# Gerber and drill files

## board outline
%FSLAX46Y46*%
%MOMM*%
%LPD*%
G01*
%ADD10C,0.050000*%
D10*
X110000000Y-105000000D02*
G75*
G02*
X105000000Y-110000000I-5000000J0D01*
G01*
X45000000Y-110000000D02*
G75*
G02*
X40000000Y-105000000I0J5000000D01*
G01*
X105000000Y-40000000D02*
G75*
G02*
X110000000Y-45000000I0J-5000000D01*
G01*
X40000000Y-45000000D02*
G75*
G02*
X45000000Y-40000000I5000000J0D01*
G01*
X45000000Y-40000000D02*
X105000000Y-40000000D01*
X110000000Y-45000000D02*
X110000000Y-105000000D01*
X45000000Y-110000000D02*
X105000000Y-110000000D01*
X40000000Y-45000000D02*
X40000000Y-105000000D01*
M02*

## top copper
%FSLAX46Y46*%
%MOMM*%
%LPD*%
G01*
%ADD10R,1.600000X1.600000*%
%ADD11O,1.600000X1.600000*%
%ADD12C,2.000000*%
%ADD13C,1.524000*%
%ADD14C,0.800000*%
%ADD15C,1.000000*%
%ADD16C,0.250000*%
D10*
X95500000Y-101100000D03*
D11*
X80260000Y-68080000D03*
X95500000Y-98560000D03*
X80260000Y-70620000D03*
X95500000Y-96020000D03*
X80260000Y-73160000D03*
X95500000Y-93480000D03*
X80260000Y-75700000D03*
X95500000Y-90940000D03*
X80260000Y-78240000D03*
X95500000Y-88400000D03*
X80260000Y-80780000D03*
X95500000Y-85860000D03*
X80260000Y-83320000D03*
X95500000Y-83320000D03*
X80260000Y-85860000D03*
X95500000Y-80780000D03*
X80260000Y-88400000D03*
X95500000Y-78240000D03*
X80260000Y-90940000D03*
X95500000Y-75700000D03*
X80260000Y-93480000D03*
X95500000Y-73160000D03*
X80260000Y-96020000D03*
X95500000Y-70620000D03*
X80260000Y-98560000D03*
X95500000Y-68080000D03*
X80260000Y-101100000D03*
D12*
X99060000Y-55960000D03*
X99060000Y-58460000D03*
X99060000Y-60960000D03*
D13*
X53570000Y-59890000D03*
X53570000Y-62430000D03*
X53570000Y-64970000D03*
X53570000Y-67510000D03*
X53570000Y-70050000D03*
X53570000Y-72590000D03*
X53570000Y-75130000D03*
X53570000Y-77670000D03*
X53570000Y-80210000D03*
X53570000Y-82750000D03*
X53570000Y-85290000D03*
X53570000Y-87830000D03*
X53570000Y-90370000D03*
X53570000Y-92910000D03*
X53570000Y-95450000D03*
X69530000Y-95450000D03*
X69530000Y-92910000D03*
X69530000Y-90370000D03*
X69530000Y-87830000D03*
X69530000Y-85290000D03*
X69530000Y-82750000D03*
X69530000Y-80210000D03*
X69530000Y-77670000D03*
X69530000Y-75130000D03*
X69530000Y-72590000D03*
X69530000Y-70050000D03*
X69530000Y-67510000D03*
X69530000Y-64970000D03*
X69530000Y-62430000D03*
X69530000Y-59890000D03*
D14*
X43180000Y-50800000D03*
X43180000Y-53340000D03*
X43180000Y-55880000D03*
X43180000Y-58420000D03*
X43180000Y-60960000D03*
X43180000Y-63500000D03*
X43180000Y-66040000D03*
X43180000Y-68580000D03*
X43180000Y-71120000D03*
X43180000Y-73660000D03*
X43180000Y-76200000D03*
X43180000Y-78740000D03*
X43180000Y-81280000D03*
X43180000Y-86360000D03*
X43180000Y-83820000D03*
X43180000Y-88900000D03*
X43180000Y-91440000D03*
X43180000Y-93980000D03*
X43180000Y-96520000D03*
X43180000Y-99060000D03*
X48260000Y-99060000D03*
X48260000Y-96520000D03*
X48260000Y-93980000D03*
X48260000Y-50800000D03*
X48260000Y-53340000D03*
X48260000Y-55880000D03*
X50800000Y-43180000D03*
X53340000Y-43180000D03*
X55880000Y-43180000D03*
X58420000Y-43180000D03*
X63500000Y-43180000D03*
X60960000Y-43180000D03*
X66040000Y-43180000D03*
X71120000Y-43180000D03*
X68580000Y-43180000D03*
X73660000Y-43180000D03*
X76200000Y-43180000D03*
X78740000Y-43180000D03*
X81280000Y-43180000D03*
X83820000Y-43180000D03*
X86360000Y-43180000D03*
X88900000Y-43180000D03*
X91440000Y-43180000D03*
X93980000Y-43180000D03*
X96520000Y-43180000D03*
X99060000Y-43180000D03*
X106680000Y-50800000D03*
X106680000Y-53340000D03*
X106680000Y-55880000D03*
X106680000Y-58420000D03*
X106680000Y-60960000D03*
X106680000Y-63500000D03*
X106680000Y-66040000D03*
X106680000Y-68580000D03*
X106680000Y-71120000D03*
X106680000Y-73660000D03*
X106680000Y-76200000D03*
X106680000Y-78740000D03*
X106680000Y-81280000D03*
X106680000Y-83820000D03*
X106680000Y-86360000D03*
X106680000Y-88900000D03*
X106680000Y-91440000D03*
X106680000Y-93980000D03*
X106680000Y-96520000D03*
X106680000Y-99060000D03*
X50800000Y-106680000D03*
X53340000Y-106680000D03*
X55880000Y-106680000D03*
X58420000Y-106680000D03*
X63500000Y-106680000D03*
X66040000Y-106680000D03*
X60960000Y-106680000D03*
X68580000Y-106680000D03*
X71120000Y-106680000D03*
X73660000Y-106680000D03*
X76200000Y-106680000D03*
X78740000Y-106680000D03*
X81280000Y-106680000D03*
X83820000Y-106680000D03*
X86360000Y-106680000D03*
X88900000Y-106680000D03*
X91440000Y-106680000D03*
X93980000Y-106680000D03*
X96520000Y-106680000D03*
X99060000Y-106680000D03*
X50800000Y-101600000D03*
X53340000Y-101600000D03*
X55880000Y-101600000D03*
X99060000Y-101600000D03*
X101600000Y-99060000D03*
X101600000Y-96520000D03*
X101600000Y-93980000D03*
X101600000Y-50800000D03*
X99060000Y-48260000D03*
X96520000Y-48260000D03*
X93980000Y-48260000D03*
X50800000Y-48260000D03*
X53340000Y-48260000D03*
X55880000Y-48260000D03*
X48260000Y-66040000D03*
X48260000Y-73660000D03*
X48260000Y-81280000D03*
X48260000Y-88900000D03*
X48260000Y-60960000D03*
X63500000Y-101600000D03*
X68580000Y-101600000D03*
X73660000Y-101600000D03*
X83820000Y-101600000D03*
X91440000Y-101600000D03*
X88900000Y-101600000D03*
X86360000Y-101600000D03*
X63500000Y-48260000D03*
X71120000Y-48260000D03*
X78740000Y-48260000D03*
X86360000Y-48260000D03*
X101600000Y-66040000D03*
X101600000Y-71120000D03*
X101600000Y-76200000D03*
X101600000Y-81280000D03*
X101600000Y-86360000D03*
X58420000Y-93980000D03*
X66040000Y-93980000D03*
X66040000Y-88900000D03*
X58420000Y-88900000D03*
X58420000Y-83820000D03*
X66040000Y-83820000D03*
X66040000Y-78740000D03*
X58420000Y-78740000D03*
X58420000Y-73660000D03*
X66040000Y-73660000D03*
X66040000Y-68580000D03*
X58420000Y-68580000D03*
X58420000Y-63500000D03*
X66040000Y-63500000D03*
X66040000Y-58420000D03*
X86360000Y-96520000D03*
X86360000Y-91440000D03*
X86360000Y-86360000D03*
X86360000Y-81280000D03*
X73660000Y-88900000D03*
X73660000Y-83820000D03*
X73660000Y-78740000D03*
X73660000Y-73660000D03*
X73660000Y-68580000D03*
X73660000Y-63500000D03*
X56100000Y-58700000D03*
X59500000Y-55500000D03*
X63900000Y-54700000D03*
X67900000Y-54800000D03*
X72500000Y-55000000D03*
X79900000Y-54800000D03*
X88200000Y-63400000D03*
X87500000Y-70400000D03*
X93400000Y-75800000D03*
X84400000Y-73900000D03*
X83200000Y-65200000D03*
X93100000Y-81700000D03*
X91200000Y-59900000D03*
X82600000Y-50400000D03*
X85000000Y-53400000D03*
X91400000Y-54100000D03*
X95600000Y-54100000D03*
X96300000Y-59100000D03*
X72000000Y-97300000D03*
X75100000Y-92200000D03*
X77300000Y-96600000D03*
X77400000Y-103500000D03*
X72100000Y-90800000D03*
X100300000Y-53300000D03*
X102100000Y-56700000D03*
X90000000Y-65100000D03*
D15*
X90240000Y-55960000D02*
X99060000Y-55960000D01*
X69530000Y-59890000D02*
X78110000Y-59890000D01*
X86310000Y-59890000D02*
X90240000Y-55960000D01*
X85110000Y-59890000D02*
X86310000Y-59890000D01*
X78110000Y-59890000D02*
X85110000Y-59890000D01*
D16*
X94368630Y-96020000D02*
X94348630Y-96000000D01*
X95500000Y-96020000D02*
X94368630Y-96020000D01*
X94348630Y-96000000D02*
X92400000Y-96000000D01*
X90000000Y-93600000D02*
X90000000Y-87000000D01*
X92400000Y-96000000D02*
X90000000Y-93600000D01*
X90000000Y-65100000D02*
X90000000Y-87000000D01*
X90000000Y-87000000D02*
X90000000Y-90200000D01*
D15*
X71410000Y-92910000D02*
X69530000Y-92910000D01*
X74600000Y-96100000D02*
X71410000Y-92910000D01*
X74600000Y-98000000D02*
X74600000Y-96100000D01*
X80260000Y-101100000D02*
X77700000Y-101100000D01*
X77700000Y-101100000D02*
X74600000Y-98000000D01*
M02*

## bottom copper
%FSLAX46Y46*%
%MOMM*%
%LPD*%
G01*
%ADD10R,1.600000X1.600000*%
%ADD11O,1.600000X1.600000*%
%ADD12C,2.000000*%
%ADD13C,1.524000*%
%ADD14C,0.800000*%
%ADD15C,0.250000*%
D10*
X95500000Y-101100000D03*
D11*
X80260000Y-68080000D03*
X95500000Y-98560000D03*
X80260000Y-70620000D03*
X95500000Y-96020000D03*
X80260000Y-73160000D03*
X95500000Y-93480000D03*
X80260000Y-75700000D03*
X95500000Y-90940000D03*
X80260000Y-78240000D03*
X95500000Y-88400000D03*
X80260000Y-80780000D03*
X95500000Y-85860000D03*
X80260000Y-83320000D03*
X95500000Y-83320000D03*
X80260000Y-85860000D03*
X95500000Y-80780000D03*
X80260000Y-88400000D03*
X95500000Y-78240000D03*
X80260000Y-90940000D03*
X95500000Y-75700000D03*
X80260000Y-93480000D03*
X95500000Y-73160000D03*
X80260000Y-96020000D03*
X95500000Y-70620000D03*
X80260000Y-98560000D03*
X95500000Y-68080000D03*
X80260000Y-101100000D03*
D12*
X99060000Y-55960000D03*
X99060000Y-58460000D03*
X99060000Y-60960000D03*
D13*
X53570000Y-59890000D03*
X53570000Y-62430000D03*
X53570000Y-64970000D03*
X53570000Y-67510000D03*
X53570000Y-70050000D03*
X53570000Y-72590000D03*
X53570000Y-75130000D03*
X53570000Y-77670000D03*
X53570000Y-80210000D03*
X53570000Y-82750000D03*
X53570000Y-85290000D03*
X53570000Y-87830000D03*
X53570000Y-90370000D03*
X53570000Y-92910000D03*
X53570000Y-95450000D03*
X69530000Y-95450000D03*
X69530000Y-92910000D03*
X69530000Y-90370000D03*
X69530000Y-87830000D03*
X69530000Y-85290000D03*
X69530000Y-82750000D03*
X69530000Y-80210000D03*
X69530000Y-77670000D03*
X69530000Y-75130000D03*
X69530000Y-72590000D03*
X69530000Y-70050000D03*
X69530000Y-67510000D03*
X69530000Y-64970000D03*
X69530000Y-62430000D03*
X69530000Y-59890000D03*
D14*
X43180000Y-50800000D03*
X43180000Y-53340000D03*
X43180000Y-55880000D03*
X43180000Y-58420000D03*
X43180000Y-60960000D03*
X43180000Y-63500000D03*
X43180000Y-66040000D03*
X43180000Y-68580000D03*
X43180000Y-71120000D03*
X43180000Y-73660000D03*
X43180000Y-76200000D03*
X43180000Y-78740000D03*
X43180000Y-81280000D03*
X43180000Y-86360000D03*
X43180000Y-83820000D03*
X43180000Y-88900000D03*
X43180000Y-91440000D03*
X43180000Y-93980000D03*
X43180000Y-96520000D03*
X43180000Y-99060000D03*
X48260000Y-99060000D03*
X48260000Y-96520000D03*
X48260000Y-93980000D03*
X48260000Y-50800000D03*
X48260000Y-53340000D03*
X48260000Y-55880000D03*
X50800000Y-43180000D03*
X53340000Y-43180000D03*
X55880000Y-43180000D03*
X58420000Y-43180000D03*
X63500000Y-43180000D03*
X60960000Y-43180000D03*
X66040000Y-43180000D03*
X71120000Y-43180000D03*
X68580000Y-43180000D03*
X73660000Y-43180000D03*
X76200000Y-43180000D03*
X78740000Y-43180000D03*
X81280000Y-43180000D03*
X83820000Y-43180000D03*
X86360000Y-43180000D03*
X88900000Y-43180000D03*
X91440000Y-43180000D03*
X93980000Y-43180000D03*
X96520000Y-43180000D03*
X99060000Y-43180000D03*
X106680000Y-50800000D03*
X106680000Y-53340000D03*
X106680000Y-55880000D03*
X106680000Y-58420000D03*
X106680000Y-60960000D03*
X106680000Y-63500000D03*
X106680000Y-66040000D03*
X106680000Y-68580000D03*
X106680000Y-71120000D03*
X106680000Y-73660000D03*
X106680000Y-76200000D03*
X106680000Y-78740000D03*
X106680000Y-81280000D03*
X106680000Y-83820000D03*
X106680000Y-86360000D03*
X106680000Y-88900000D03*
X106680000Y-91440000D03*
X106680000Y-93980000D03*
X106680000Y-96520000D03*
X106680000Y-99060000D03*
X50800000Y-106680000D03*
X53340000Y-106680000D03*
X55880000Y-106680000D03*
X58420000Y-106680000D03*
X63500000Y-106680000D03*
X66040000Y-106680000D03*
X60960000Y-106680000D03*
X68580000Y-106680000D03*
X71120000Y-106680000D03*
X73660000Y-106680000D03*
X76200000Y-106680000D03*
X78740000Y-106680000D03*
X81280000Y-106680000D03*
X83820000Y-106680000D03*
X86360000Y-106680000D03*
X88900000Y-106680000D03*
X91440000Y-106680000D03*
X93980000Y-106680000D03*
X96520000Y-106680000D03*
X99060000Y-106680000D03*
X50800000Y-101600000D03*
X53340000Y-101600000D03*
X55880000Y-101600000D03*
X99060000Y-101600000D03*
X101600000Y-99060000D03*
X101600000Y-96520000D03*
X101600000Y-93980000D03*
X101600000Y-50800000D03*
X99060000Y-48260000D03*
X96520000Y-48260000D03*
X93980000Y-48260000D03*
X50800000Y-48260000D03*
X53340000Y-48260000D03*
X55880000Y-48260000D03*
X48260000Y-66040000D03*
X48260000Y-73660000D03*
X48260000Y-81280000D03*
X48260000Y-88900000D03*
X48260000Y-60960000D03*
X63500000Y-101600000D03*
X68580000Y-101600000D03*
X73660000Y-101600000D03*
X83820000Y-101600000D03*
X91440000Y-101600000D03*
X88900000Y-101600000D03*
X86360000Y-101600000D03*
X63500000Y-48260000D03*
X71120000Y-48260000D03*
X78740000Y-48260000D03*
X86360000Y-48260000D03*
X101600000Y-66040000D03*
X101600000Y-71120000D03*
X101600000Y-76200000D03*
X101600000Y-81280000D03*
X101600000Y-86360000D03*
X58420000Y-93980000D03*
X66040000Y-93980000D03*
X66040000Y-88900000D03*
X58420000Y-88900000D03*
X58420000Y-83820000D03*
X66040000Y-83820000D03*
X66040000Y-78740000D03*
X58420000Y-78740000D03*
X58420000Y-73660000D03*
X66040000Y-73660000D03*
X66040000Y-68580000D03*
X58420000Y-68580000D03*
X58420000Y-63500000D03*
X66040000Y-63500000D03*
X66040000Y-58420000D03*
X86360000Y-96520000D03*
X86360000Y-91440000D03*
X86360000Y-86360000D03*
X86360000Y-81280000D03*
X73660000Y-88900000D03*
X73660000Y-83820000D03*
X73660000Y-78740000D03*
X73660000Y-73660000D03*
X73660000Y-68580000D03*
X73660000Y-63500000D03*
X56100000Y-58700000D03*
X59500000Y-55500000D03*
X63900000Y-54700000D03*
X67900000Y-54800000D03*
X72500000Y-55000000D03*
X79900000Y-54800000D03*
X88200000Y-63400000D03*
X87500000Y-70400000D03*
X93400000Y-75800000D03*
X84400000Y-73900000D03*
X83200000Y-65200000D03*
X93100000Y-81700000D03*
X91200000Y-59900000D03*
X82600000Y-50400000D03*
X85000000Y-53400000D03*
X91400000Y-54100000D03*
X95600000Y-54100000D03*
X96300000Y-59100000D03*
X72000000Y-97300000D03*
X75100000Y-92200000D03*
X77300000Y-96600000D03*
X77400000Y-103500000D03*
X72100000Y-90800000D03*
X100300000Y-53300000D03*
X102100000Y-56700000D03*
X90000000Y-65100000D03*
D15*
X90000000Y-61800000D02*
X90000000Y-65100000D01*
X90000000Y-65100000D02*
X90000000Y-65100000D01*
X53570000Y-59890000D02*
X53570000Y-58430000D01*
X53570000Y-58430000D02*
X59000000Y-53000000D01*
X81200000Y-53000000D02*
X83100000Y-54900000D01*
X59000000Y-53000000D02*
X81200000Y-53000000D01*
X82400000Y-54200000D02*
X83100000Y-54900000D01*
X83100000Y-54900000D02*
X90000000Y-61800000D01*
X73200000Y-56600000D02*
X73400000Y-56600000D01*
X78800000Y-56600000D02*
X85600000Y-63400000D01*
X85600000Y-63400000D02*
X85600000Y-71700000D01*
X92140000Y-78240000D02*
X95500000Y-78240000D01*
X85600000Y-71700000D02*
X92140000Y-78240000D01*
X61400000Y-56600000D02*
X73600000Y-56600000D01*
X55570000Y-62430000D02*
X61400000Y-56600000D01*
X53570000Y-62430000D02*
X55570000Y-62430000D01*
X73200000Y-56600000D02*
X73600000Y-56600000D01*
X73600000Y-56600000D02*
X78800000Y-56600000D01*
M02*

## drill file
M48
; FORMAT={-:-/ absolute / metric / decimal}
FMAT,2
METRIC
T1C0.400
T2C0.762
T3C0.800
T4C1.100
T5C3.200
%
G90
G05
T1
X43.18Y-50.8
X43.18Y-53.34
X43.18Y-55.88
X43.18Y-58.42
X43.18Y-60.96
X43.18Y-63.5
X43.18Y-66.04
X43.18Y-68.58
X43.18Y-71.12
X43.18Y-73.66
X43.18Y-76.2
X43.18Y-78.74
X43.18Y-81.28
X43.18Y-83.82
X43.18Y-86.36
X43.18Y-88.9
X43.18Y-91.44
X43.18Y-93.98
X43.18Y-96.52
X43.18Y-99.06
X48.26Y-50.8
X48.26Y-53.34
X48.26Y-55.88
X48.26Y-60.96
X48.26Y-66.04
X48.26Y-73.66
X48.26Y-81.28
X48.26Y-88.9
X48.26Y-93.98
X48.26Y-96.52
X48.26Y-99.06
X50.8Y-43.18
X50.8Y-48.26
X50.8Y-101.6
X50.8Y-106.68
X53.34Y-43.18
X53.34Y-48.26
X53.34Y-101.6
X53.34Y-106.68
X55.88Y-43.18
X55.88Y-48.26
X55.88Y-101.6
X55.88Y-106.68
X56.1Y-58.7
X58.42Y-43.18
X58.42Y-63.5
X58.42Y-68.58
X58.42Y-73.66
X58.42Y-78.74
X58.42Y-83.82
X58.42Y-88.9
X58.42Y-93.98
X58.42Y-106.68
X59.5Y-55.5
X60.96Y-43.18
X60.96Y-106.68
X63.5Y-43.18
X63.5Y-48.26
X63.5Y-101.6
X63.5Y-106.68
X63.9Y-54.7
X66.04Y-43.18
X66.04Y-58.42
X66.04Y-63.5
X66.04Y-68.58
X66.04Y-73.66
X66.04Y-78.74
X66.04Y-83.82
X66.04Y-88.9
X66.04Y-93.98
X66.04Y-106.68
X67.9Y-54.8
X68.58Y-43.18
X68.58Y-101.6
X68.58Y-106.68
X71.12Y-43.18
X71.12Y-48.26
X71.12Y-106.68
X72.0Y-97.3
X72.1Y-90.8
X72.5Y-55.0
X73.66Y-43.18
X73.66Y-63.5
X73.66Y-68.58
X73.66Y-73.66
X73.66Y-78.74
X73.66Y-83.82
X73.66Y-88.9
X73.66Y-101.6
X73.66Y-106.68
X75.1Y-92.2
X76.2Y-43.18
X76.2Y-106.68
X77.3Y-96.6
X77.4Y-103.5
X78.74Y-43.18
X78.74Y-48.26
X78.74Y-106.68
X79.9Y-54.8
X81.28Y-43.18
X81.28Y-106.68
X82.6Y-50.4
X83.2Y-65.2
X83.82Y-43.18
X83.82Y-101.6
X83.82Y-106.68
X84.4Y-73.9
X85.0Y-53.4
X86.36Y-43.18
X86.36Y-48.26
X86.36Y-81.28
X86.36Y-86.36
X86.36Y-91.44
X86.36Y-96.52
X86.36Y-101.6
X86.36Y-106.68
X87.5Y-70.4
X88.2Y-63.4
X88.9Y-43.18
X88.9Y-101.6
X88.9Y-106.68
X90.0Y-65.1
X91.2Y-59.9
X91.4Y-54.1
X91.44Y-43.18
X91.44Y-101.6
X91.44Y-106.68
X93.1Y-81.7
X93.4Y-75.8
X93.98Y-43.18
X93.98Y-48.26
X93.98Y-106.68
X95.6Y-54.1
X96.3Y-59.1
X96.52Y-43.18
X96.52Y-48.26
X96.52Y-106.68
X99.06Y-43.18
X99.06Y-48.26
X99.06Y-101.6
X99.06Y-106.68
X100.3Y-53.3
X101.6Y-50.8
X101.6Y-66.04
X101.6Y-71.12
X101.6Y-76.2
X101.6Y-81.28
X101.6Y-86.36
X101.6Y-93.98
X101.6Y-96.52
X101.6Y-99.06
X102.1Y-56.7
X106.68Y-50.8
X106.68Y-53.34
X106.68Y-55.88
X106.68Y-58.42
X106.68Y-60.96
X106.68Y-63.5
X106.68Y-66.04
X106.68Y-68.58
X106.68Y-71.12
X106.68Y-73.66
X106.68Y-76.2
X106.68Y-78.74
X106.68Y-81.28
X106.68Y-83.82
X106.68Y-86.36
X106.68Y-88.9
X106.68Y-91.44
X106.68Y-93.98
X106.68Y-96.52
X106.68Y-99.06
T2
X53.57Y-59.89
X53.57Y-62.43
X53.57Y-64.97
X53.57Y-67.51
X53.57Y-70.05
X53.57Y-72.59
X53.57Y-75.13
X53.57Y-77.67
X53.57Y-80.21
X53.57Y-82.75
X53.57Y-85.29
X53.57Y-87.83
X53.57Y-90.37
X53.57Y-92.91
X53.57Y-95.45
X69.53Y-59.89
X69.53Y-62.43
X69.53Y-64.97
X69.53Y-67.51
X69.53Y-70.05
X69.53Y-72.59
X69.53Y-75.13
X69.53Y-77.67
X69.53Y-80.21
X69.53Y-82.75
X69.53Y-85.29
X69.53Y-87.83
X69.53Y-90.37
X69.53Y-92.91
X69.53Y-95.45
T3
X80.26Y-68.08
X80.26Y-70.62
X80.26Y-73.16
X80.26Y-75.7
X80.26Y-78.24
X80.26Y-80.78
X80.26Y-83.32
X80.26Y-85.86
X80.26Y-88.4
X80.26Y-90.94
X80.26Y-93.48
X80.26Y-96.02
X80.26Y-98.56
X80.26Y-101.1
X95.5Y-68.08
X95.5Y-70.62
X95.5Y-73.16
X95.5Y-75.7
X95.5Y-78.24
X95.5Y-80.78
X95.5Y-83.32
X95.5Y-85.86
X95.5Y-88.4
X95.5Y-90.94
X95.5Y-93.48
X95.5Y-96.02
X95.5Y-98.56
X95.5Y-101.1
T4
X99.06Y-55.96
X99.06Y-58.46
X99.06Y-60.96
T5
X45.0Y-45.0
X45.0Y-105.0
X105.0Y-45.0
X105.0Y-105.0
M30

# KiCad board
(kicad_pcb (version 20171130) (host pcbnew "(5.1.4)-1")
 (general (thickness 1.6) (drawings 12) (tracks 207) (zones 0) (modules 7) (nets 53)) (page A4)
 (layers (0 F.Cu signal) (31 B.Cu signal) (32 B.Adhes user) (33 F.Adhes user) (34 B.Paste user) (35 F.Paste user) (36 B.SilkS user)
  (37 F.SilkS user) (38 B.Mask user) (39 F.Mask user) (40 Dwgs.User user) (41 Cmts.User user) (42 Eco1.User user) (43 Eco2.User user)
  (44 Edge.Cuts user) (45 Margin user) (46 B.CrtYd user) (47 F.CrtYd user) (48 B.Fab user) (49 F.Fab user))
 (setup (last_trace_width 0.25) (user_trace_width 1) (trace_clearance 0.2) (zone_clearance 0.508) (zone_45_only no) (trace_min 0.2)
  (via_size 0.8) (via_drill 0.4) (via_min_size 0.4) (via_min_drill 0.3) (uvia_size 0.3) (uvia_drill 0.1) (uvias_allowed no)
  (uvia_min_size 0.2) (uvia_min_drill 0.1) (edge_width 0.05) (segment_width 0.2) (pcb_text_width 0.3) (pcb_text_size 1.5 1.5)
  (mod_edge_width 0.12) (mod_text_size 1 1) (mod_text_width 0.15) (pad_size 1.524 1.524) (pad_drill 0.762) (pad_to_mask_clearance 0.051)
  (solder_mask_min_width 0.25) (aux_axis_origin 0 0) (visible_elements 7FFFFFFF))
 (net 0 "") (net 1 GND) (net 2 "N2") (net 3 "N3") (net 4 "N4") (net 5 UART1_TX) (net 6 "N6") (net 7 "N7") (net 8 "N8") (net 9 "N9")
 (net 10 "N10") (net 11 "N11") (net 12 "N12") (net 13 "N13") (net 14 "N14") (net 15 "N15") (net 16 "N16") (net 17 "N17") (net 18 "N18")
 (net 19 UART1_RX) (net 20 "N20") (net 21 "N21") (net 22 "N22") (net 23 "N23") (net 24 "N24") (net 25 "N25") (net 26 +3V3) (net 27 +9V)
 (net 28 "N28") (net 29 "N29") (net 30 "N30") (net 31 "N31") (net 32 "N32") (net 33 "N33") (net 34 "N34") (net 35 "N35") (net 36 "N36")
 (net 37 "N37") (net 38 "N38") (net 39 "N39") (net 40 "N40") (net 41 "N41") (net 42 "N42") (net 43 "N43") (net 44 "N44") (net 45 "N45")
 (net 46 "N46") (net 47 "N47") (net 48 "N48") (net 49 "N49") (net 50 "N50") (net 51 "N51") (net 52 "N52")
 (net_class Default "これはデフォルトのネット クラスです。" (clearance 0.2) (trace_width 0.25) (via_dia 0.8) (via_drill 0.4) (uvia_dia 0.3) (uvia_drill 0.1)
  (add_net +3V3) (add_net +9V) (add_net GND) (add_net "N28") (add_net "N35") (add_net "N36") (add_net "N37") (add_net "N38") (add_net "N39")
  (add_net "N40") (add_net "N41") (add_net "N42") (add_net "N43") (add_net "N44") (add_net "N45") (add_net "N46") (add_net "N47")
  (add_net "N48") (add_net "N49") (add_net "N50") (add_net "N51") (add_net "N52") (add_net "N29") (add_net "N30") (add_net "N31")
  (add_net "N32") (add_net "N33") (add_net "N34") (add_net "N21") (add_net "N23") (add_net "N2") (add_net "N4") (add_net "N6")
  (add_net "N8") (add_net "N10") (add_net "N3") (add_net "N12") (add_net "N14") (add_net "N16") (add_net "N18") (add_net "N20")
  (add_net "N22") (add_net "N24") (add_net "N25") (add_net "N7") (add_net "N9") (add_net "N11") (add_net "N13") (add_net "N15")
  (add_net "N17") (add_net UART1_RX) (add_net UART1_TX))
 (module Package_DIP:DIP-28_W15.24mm (layer F.Cu) (at 95.5 101.1 180)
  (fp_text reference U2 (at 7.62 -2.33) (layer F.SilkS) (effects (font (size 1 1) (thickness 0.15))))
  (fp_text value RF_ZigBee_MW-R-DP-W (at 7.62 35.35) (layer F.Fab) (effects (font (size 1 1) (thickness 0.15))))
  (pad 1 thru_hole rect (at 0 0 180) (size 1.6 1.6) (drill 0.8) (layers *.Cu *.Mask) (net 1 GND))
  (pad 15 thru_hole oval (at 15.24 33.02 180) (size 1.6 1.6) (drill 0.8) (layers *.Cu *.Mask) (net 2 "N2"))
  (pad 2 thru_hole oval (at 0 2.54 180) (size 1.6 1.6) (drill 0.8) (layers *.Cu *.Mask) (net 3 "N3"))
  (pad 16 thru_hole oval (at 15.24 30.48 180) (size 1.6 1.6) (drill 0.8) (layers *.Cu *.Mask) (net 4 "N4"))
  (pad 3 thru_hole oval (at 0 5.08 180) (size 1.6 1.6) (drill 0.8) (layers *.Cu *.Mask) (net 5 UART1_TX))
  (pad 17 thru_hole oval (at 15.24 27.94 180) (size 1.6 1.6) (drill 0.8) (layers *.Cu *.Mask) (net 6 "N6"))
  (pad 4 thru_hole oval (at 0 7.62 180) (size 1.6 1.6) (drill 0.8) (layers *.Cu *.Mask) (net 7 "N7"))
  (pad 18 thru_hole oval (at 15.24 25.4 180) (size 1.6 1.6) (drill 0.8) (layers *.Cu *.Mask) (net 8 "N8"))
  (pad 5 thru_hole oval (at 0 10.16 180) (size 1.6 1.6) (drill 0.8) (layers *.Cu *.Mask) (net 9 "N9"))
  (pad 19 thru_hole oval (at 15.24 22.86 180) (size 1.6 1.6) (drill 0.8) (layers *.Cu *.Mask) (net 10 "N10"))
  (pad 6 thru_hole oval (at 0 12.7 180) (size 1.6 1.6) (drill 0.8) (layers *.Cu *.Mask) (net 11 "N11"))
  (pad 20 thru_hole oval (at 15.24 20.32 180) (size 1.6 1.6) (drill 0.8) (layers *.Cu *.Mask) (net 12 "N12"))
  (pad 7 thru_hole oval (at 0 15.24 180) (size 1.6 1.6) (drill 0.8) (layers *.Cu *.Mask) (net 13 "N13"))
  (pad 21 thru_hole oval (at 15.24 17.78 180) (size 1.6 1.6) (drill 0.8) (layers *.Cu *.Mask) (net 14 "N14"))
  (pad 8 thru_hole oval (at 0 17.78 180) (size 1.6 1.6) (drill 0.8) (layers *.Cu *.Mask) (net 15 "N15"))
  (pad 22 thru_hole oval (at 15.24 15.24 180) (size 1.6 1.6) (drill 0.8) (layers *.Cu *.Mask) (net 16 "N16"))
  (pad 9 thru_hole oval (at 0 20.32 180) (size 1.6 1.6) (drill 0.8) (layers *.Cu *.Mask) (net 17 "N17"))
  (pad 23 thru_hole oval (at 15.24 12.7 180) (size 1.6 1.6) (drill 0.8) (layers *.Cu *.Mask) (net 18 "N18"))
  (pad 10 thru_hole oval (at 0 22.86 180) (size 1.6 1.6) (drill 0.8) (layers *.Cu *.Mask) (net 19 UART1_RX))
  (pad 24 thru_hole oval (at 15.24 10.16 180) (size 1.6 1.6) (drill 0.8) (layers *.Cu *.Mask) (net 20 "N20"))
  (pad 11 thru_hole oval (at 0 25.4 180) (size 1.6 1.6) (drill 0.8) (layers *.Cu *.Mask) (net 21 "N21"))
  (pad 25 thru_hole oval (at 15.24 7.62 180) (size 1.6 1.6) (drill 0.8) (layers *.Cu *.Mask) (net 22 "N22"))
  (pad 12 thru_hole oval (at 0 27.94 180) (size 1.6 1.6) (drill 0.8) (layers *.Cu *.Mask) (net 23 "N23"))
  (pad 26 thru_hole oval (at 15.24 5.08 180) (size 1.6 1.6) (drill 0.8) (layers *.Cu *.Mask) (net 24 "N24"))
  (pad 13 thru_hole oval (at 0 30.48 180) (size 1.6 1.6) (drill 0.8) (layers *.Cu *.Mask) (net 1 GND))
  (pad 27 thru_hole oval (at 15.24 2.54 180) (size 1.6 1.6) (drill 0.8) (layers *.Cu *.Mask) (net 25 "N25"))
  (pad 14 thru_hole oval (at 0 33.02 180) (size 1.6 1.6) (drill 0.8) (layers *.Cu *.Mask) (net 1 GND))
  (pad 28 thru_hole oval (at 15.24 0 180) (size 1.6 1.6) (drill 0.8) (layers *.Cu *.Mask) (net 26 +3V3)))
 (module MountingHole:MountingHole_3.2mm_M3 (layer F.Cu) (at 45 45)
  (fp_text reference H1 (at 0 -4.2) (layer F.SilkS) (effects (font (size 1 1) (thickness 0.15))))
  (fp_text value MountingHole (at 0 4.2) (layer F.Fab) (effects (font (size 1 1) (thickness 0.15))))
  (pad 1 np_thru_hole circle (at 0 0) (size 3.2 3.2) (drill 3.2) (layers *.Cu *.Mask)))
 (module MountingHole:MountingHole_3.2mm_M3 (layer F.Cu) (at 105 45)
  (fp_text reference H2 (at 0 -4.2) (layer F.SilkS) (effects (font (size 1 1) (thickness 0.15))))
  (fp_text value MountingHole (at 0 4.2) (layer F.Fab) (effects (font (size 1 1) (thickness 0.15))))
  (pad 1 np_thru_hole circle (at 0 0) (size 3.2 3.2) (drill 3.2) (layers *.Cu *.Mask)))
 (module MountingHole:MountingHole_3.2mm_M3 (layer F.Cu) (at 45 105)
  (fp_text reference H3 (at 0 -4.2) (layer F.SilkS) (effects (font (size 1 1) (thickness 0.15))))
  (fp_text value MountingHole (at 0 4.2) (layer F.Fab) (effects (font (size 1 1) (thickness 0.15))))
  (pad 1 np_thru_hole circle (at 0 0) (size 3.2 3.2) (drill 3.2) (layers *.Cu *.Mask)))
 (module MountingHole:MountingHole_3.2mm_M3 (layer F.Cu) (at 105 105)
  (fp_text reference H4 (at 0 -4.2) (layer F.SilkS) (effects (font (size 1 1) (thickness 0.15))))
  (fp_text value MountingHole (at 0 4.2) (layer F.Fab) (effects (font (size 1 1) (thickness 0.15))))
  (pad 1 np_thru_hole circle (at 0 0) (size 3.2 3.2) (drill 3.2) (layers *.Cu *.Mask)))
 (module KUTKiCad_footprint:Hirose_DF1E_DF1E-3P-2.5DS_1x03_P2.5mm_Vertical (layer F.Cu) (at 99.06 55.96 270)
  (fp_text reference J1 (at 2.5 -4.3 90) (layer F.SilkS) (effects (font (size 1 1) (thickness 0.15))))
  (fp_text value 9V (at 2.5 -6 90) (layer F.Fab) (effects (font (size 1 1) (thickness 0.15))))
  (pad 1 thru_hole circle (at 0 0 270) (size 2 2) (drill 1.1) (layers *.Cu *.Mask) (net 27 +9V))
  (pad 2 thru_hole circle (at 2.5 0 270) (size 2 2) (drill 1.1) (layers *.Cu *.Mask) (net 1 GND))
  (pad 3 thru_hole circle (at 5 0 270) (size 2 2) (drill 1.1) (layers *.Cu *.Mask) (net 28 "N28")))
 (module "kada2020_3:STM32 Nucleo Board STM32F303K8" (layer F.Cu) (at 52.3 51)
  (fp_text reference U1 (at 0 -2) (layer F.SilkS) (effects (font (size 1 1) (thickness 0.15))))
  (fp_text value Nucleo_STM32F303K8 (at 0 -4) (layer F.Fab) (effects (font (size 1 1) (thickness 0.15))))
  (pad 1 thru_hole circle (at 1.27 8.89) (size 1.524 1.524) (drill 0.762) (layers *.Cu *.Mask) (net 5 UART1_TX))
  (pad 2 thru_hole circle (at 1.27 11.43) (size 1.524 1.524) (drill 0.762) (layers *.Cu *.Mask) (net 19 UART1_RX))
  (pad 3 thru_hole circle (at 1.27 13.97) (size 1.524 1.524) (drill 0.762) (layers *.Cu *.Mask) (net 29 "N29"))
  (pad 4 thru_hole circle (at 1.27 16.51) (size 1.524 1.524) (drill 0.762) (layers *.Cu *.Mask) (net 1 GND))
  (pad 5 thru_hole circle (at 1.27 19.05) (size 1.524 1.524) (drill 0.762) (layers *.Cu *.Mask) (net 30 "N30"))
  (pad 6 thru_hole circle (at 1.27 21.59) (size 1.524 1.524) (drill 0.762) (layers *.Cu *.Mask) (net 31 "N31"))
  (pad 7 thru_hole circle (at 1.27 24.13) (size 1.524 1.524) (drill 0.762) (layers *.Cu *.Mask) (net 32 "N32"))
  (pad 8 thru_hole circle (at 1.27 26.67) (size 1.524 1.524) (drill 0.762) (layers *.Cu *.Mask) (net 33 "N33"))
  (pad 9 thru_hole circle (at 1.27 29.21) (size 1.524 1.524) (drill 0.762) (layers *.Cu *.Mask) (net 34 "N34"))
  (pad 10 thru_hole circle (at 1.27 31.75) (size 1.524 1.524) (drill 0.762) (layers *.Cu *.Mask) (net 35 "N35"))
  (pad 11 thru_hole circle (at 1.27 34.29) (size 1.524 1.524) (drill 0.762) (layers *.Cu *.Mask) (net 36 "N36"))
  (pad 12 thru_hole circle (at 1.27 36.83) (size 1.524 1.524) (drill 0.762) (layers *.Cu *.Mask) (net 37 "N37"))
  (pad 13 thru_hole circle (at 1.27 39.37) (size 1.524 1.524) (drill 0.762) (layers *.Cu *.Mask) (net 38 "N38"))
  (pad 14 thru_hole circle (at 1.27 41.91) (size 1.524 1.524) (drill 0.762) (layers *.Cu *.Mask) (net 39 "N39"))
  (pad 15 thru_hole circle (at 1.27 44.45) (size 1.524 1.524) (drill 0.762) (layers *.Cu *.Mask) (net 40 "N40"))
  (pad 16 thru_hole circle (at 17.23 44.45) (size 1.524 1.524) (drill 0.762) (layers *.Cu *.Mask) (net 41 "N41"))
  (pad 17 thru_hole circle (at 17.23 41.91) (size 1.524 1.524) (drill 0.762) (layers *.Cu *.Mask) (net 26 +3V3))
  (pad 18 thru_hole circle (at 17.23 39.37) (size 1.524 1.524) (drill 0.762) (layers *.Cu *.Mask) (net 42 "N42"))
  (pad 19 thru_hole circle (at 17.23 36.83) (size 1.524 1.524) (drill 0.762) (layers *.Cu *.Mask) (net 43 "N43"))
  (pad 20 thru_hole circle (at 17.23 34.29) (size 1.524 1.524) (drill 0.762) (layers *.Cu *.Mask) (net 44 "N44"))
  (pad 21 thru_hole circle (at 17.23 31.75) (size 1.524 1.524) (drill 0.762) (layers *.Cu *.Mask) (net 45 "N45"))
  (pad 22 thru_hole circle (at 17.23 29.21) (size 1.524 1.524) (drill 0.762) (layers *.Cu *.Mask) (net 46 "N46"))
  (pad 23 thru_hole circle (at 17.23 26.67) (size 1.524 1.524) (drill 0.762) (layers *.Cu *.Mask) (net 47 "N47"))
  (pad 24 thru_hole circle (at 17.23 24.13) (size 1.524 1.524) (drill 0.762) (layers *.Cu *.Mask) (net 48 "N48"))
  (pad 25 thru_hole circle (at 17.23 21.59) (size 1.524 1.524) (drill 0.762) (layers *.Cu *.Mask) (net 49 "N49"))
  (pad 26 thru_hole circle (at 17.23 19.05) (size 1.524 1.524) (drill 0.762) (layers *.Cu *.Mask) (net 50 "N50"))
  (pad 27 thru_hole circle (at 17.23 16.51) (size 1.524 1.524) (drill 0.762) (layers *.Cu *.Mask) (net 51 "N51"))
  (pad 28 thru_hole circle (at 17.23 13.97) (size 1.524 1.524) (drill 0.762) (layers *.Cu *.Mask) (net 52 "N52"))
  (pad 29 thru_hole circle (at 17.23 11.43) (size 1.524 1.524) (drill 0.762) (layers *.Cu *.Mask) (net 1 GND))
  (pad 30 thru_hole circle (at 17.23 8.89) (size 1.524 1.524) (drill 0.762) (layers *.Cu *.Mask) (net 27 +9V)))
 (gr_arc (start 105 105) (end 105 110) (angle -90) (layer Edge.Cuts) (width 0.05))
 (gr_arc (start 45 105) (end 40 105) (angle -90) (layer Edge.Cuts) (width 0.05))
 (gr_arc (start 105 45) (end 110 45) (angle -90) (layer Edge.Cuts) (width 0.05))
 (gr_arc (start 45 45) (end 45 40) (angle -90) (layer Edge.Cuts) (width 0.05))
 (gr_line (start 45 40) (end 105 40) (layer Edge.Cuts) (width 0.05))
 (gr_line (start 110 45) (end 110 105) (layer Edge.Cuts) (width 0.05))
 (gr_line (start 45 110) (end 105 110) (layer Edge.Cuts) (width 0.05))
 (gr_line (start 40 45) (end 40 105) (layer Edge.Cuts) (width 0.05))
 (segment (start 90.24 55.96) (end 99.06 55.96) (width 1) (layer F.Cu) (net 27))
 (segment (start 69.53 59.89) (end 78.11 59.89) (width 1) (layer F.Cu) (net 27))
 (segment (start 86.31 59.89) (end 90.24 55.96) (width 1) (layer F.Cu) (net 27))
 (segment (start 85.11 59.89) (end 86.31 59.89) (width 1) (layer F.Cu) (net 27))
 (segment (start 78.11 59.89) (end 85.11 59.89) (width 1) (layer F.Cu) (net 27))
 (via (at 43.18 50.8) (size 0.8) (drill 0.4) (layers F.Cu B.Cu) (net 1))
 (via (at 43.18 53.34) (size 0.8) (drill 0.4) (layers F.Cu B.Cu) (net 1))
 (via (at 43.18 55.88) (size 0.8) (drill 0.4) (layers F.Cu B.Cu) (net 1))
 (via (at 43.18 58.42) (size 0.8) (drill 0.4) (layers F.Cu B.Cu) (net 1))
 (via (at 43.18 60.96) (size 0.8) (drill 0.4) (layers F.Cu B.Cu) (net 1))
 (via (at 43.18 63.5) (size 0.8) (drill 0.4) (layers F.Cu B.Cu) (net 1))
 (via (at 43.18 66.04) (size 0.8) (drill 0.4) (layers F.Cu B.Cu) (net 1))
 (via (at 43.18 68.58) (size 0.8) (drill 0.4) (layers F.Cu B.Cu) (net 1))
 (via (at 43.18 71.12) (size 0.8) (drill 0.4) (layers F.Cu B.Cu) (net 1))
 (via (at 43.18 73.66) (size 0.8) (drill 0.4) (layers F.Cu B.Cu) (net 1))
 (via (at 43.18 76.2) (size 0.8) (drill 0.4) (layers F.Cu B.Cu) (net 1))
 (via (at 43.18 78.74) (size 0.8) (drill 0.4) (layers F.Cu B.Cu) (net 1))
 (via (at 43.18 81.28) (size 0.8) (drill 0.4) (layers F.Cu B.Cu) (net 1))
 (via (at 43.18 86.36) (size 0.8) (drill 0.4) (layers F.Cu B.Cu) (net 1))
 (via (at 43.18 83.82) (size 0.8) (drill 0.4) (layers F.Cu B.Cu) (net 1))
 (via (at 43.18 88.9) (size 0.8) (drill 0.4) (layers F.Cu B.Cu) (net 1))
 (via (at 43.18 91.44) (size 0.8) (drill 0.4) (layers F.Cu B.Cu) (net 1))
 (via (at 43.18 93.98) (size 0.8) (drill 0.4) (layers F.Cu B.Cu) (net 1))
 (via (at 43.18 96.52) (size 0.8) (drill 0.4) (layers F.Cu B.Cu) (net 1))
 (via (at 43.18 99.06) (size 0.8) (drill 0.4) (layers F.Cu B.Cu) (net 1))
 (via (at 48.26 99.06) (size 0.8) (drill 0.4) (layers F.Cu B.Cu) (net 1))
 (via (at 48.26 96.52) (size 0.8) (drill 0.4) (layers F.Cu B.Cu) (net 1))
 (via (at 48.26 93.98) (size 0.8) (drill 0.4) (layers F.Cu B.Cu) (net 1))
 (via (at 48.26 50.8) (size 0.8) (drill 0.4) (layers F.Cu B.Cu) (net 1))
 (via (at 48.26 53.34) (size 0.8) (drill 0.4) (layers F.Cu B.Cu) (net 1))
 (via (at 48.26 55.88) (size 0.8) (drill 0.4) (layers F.Cu B.Cu) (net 1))
 (via (at 50.8 43.18) (size 0.8) (drill 0.4) (layers F.Cu B.Cu) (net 1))
 (via (at 53.34 43.18) (size 0.8) (drill 0.4) (layers F.Cu B.Cu) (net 1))
 (via (at 55.88 43.18) (size 0.8) (drill 0.4) (layers F.Cu B.Cu) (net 1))
 (via (at 58.42 43.18) (size 0.8) (drill 0.4) (layers F.Cu B.Cu) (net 1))
 (via (at 63.5 43.18) (size 0.8) (drill 0.4) (layers F.Cu B.Cu) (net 1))
 (via (at 60.96 43.18) (size 0.8) (drill 0.4) (layers F.Cu B.Cu) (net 1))
 (via (at 66.04 43.18) (size 0.8) (drill 0.4) (layers F.Cu B.Cu) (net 1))
 (via (at 71.12 43.18) (size 0.8) (drill 0.4) (layers F.Cu B.Cu) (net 1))
 (via (at 68.58 43.18) (size 0.8) (drill 0.4) (layers F.Cu B.Cu) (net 1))
 (via (at 73.66 43.18) (size 0.8) (drill 0.4) (layers F.Cu B.Cu) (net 1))
 (via (at 76.2 43.18) (size 0.8) (drill 0.4) (layers F.Cu B.Cu) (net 1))
 (via (at 78.74 43.18) (size 0.8) (drill 0.4) (layers F.Cu B.Cu) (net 1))
 (via (at 81.28 43.18) (size 0.8) (drill 0.4) (layers F.Cu B.Cu) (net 1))
 (via (at 83.82 43.18) (size 0.8) (drill 0.4) (layers F.Cu B.Cu) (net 1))
 (via (at 86.36 43.18) (size 0.8) (drill 0.4) (layers F.Cu B.Cu) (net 1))
 (via (at 88.9 43.18) (size 0.8) (drill 0.4) (layers F.Cu B.Cu) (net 1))
 (via (at 91.44 43.18) (size 0.8) (drill 0.4) (layers F.Cu B.Cu) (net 1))
 (via (at 93.98 43.18) (size 0.8) (drill 0.4) (layers F.Cu B.Cu) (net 1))
 (via (at 96.52 43.18) (size 0.8) (drill 0.4) (layers F.Cu B.Cu) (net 1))
 (via (at 99.06 43.18) (size 0.8) (drill 0.4) (layers F.Cu B.Cu) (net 1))
 (via (at 106.68 50.8) (size 0.8) (drill 0.4) (layers F.Cu B.Cu) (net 1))
 (via (at 106.68 53.34) (size 0.8) (drill 0.4) (layers F.Cu B.Cu) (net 1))
 (via (at 106.68 55.88) (size 0.8) (drill 0.4) (layers F.Cu B.Cu) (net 1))
 (via (at 106.68 58.42) (size 0.8) (drill 0.4) (layers F.Cu B.Cu) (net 1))
 (via (at 106.68 60.96) (size 0.8) (drill 0.4) (layers F.Cu B.Cu) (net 1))
 (via (at 106.68 63.5) (size 0.8) (drill 0.4) (layers F.Cu B.Cu) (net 1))
 (via (at 106.68 66.04) (size 0.8) (drill 0.4) (layers F.Cu B.Cu) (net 1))
 (via (at 106.68 68.58) (size 0.8) (drill 0.4) (layers F.Cu B.Cu) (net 1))
 (via (at 106.68 71.12) (size 0.8) (drill 0.4) (layers F.Cu B.Cu) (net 1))
 (via (at 106.68 73.66) (size 0.8) (drill 0.4) (layers F.Cu B.Cu) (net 1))
 (via (at 106.68 76.2) (size 0.8) (drill 0.4) (layers F.Cu B.Cu) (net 1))
 (via (at 106.68 78.74) (size 0.8) (drill 0.4) (layers F.Cu B.Cu) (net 1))
 (via (at 106.68 81.28) (size 0.8) (drill 0.4) (layers F.Cu B.Cu) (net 1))
 (via (at 106.68 83.82) (size 0.8) (drill 0.4) (layers F.Cu B.Cu) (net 1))
 (via (at 106.68 86.36) (size 0.8) (drill 0.4) (layers F.Cu B.Cu) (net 1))
 (via (at 106.68 88.9) (size 0.8) (drill 0.4) (layers F.Cu B.Cu) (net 1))
 (via (at 106.68 91.44) (size 0.8) (drill 0.4) (layers F.Cu B.Cu) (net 1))
 (via (at 106.68 93.98) (size 0.8) (drill 0.4) (layers F.Cu B.Cu) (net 1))
 (via (at 106.68 96.52) (size 0.8) (drill 0.4) (layers F.Cu B.Cu) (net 1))
 (via (at 106.68 99.06) (size 0.8) (drill 0.4) (layers F.Cu B.Cu) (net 1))
 (via (at 50.8 106.68) (size 0.8) (drill 0.4) (layers F.Cu B.Cu) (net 1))
 (via (at 53.34 106.68) (size 0.8) (drill 0.4) (layers F.Cu B.Cu) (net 1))
 (via (at 55.88 106.68) (size 0.8) (drill 0.4) (layers F.Cu B.Cu) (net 1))
 (via (at 58.42 106.68) (size 0.8) (drill 0.4) (layers F.Cu B.Cu) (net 1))
 (via (at 63.5 106.68) (size 0.8) (drill 0.4) (layers F.Cu B.Cu) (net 1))
 (via (at 66.04 106.68) (size 0.8) (drill 0.4) (layers F.Cu B.Cu) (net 1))
 (via (at 60.96 106.68) (size 0.8) (drill 0.4) (layers F.Cu B.Cu) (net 1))
 (via (at 68.58 106.68) (size 0.8) (drill 0.4) (layers F.Cu B.Cu) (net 1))
 (via (at 71.12 106.68) (size 0.8) (drill 0.4) (layers F.Cu B.Cu) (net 1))
 (via (at 73.66 106.68) (size 0.8) (drill 0.4) (layers F.Cu B.Cu) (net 1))
 (via (at 76.2 106.68) (size 0.8) (drill 0.4) (layers F.Cu B.Cu) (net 1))
 (via (at 78.74 106.68) (size 0.8) (drill 0.4) (layers F.Cu B.Cu) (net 1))
 (via (at 81.28 106.68) (size 0.8) (drill 0.4) (layers F.Cu B.Cu) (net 1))
 (via (at 83.82 106.68) (size 0.8) (drill 0.4) (layers F.Cu B.Cu) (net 1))
 (via (at 86.36 106.68) (size 0.8) (drill 0.4) (layers F.Cu B.Cu) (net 1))
 (via (at 88.9 106.68) (size 0.8) (drill 0.4) (layers F.Cu B.Cu) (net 1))
 (via (at 91.44 106.68) (size 0.8) (drill 0.4) (layers F.Cu B.Cu) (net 1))
 (via (at 93.98 106.68) (size 0.8) (drill 0.4) (layers F.Cu B.Cu) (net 1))
 (via (at 96.52 106.68) (size 0.8) (drill 0.4) (layers F.Cu B.Cu) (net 1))
 (via (at 99.06 106.68) (size 0.8) (drill 0.4) (layers F.Cu B.Cu) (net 1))
 (via (at 50.8 101.6) (size 0.8) (drill 0.4) (layers F.Cu B.Cu) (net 1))
 (via (at 53.34 101.6) (size 0.8) (drill 0.4) (layers F.Cu B.Cu) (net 1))
 (via (at 55.88 101.6) (size 0.8) (drill 0.4) (layers F.Cu B.Cu) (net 1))
 (via (at 99.06 101.6) (size 0.8) (drill 0.4) (layers F.Cu B.Cu) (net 1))
 (via (at 101.6 99.06) (size 0.8) (drill 0.4) (layers F.Cu B.Cu) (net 1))
 (via (at 101.6 96.52) (size 0.8) (drill 0.4) (layers F.Cu B.Cu) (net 1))
 (via (at 101.6 93.98) (size 0.8) (drill 0.4) (layers F.Cu B.Cu) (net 1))
 (via (at 101.6 50.8) (size 0.8) (drill 0.4) (layers F.Cu B.Cu) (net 1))
 (via (at 99.06 48.26) (size 0.8) (drill 0.4) (layers F.Cu B.Cu) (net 1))
 (via (at 96.52 48.26) (size 0.8) (drill 0.4) (layers F.Cu B.Cu) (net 1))
 (via (at 93.98 48.26) (size 0.8) (drill 0.4) (layers F.Cu B.Cu) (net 1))
 (via (at 50.8 48.26) (size 0.8) (drill 0.4) (layers F.Cu B.Cu) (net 1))
 (via (at 53.34 48.26) (size 0.8) (drill 0.4) (layers F.Cu B.Cu) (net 1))
 (via (at 55.88 48.26) (size 0.8) (drill 0.4) (layers F.Cu B.Cu) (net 1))
 (via (at 48.26 66.04) (size 0.8) (drill 0.4) (layers F.Cu B.Cu) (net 1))
 (via (at 48.26 73.66) (size 0.8) (drill 0.4) (layers F.Cu B.Cu) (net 1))
 (via (at 48.26 81.28) (size 0.8) (drill 0.4) (layers F.Cu B.Cu) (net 1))
 (via (at 48.26 88.9) (size 0.8) (drill 0.4) (layers F.Cu B.Cu) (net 1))
 (via (at 48.26 60.96) (size 0.8) (drill 0.4) (layers F.Cu B.Cu) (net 1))
 (via (at 63.5 101.6) (size 0.8) (drill 0.4) (layers F.Cu B.Cu) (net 1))
 (via (at 68.58 101.6) (size 0.8) (drill 0.4) (layers F.Cu B.Cu) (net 1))
 (via (at 73.66 101.6) (size 0.8) (drill 0.4) (layers F.Cu B.Cu) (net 1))
 (via (at 83.82 101.6) (size 0.8) (drill 0.4) (layers F.Cu B.Cu) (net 1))
 (via (at 91.44 101.6) (size 0.8) (drill 0.4) (layers F.Cu B.Cu) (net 1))
 (via (at 88.9 101.6) (size 0.8) (drill 0.4) (layers F.Cu B.Cu) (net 1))
 (via (at 86.36 101.6) (size 0.8) (drill 0.4) (layers F.Cu B.Cu) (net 1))
 (via (at 63.5 48.26) (size 0.8) (drill 0.4) (layers F.Cu B.Cu) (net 1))
 (via (at 71.12 48.26) (size 0.8) (drill 0.4) (layers F.Cu B.Cu) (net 1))
 (via (at 78.74 48.26) (size 0.8) (drill 0.4) (layers F.Cu B.Cu) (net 1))
 (via (at 86.36 48.26) (size 0.8) (drill 0.4) (layers F.Cu B.Cu) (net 1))
 (via (at 101.6 66.04) (size 0.8) (drill 0.4) (layers F.Cu B.Cu) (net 1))
 (via (at 101.6 71.12) (size 0.8) (drill 0.4) (layers F.Cu B.Cu) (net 1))
 (via (at 101.6 76.2) (size 0.8) (drill 0.4) (layers F.Cu B.Cu) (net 1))
 (via (at 101.6 81.28) (size 0.8) (drill 0.4) (layers F.Cu B.Cu) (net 1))
 (via (at 101.6 86.36) (size 0.8) (drill 0.4) (layers F.Cu B.Cu) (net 1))
 (via (at 58.42 93.98) (size 0.8) (drill 0.4) (layers F.Cu B.Cu) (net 1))
 (via (at 66.04 93.98) (size 0.8) (drill 0.4) (layers F.Cu B.Cu) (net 1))
 (via (at 66.04 88.9) (size 0.8) (drill 0.4) (layers F.Cu B.Cu) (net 1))
 (via (at 58.42 88.9) (size 0.8) (drill 0.4) (layers F.Cu B.Cu) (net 1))
 (via (at 58.42 83.82) (size 0.8) (drill 0.4) (layers F.Cu B.Cu) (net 1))
 (via (at 66.04 83.82) (size 0.8) (drill 0.4) (layers F.Cu B.Cu) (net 1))
 (via (at 66.04 78.74) (size 0.8) (drill 0.4) (layers F.Cu B.Cu) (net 1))
 (via (at 58.42 78.74) (size 0.8) (drill 0.4) (layers F.Cu B.Cu) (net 1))
 (via (at 58.42 73.66) (size 0.8) (drill 0.4) (layers F.Cu B.Cu) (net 1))
 (via (at 66.04 73.66) (size 0.8) (drill 0.4) (layers F.Cu B.Cu) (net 1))
 (via (at 66.04 68.58) (size 0.8) (drill 0.4) (layers F.Cu B.Cu) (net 1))
 (via (at 58.42 68.58) (size 0.8) (drill 0.4) (layers F.Cu B.Cu) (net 1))
 (via (at 58.42 63.5) (size 0.8) (drill 0.4) (layers F.Cu B.Cu) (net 1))
 (via (at 66.04 63.5) (size 0.8) (drill 0.4) (layers F.Cu B.Cu) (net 1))
 (via (at 66.04 58.42) (size 0.8) (drill 0.4) (layers F.Cu B.Cu) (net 1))
 (via (at 86.36 96.52) (size 0.8) (drill 0.4) (layers F.Cu B.Cu) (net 1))
 (via (at 86.36 91.44) (size 0.8) (drill 0.4) (layers F.Cu B.Cu) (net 1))
 (via (at 86.36 86.36) (size 0.8) (drill 0.4) (layers F.Cu B.Cu) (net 1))
 (via (at 86.36 81.28) (size 0.8) (drill 0.4) (layers F.Cu B.Cu) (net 1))
 (via (at 73.66 88.9) (size 0.8) (drill 0.4) (layers F.Cu B.Cu) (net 1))
 (via (at 73.66 83.82) (size 0.8) (drill 0.4) (layers F.Cu B.Cu) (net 1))
 (via (at 73.66 78.74) (size 0.8) (drill 0.4) (layers F.Cu B.Cu) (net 1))
 (via (at 73.66 73.66) (size 0.8) (drill 0.4) (layers F.Cu B.Cu) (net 1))
 (via (at 73.66 68.58) (size 0.8) (drill 0.4) (layers F.Cu B.Cu) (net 1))
 (via (at 73.66 63.5) (size 0.8) (drill 0.4) (layers F.Cu B.Cu) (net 1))
 (via (at 56.1 58.7) (size 0.8) (drill 0.4) (layers F.Cu B.Cu) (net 1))
 (via (at 59.5 55.5) (size 0.8) (drill 0.4) (layers F.Cu B.Cu) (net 1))
 (via (at 63.9 54.7) (size 0.8) (drill 0.4) (layers F.Cu B.Cu) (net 1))
 (via (at 67.9 54.8) (size 0.8) (drill 0.4) (layers F.Cu B.Cu) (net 1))
 (via (at 72.5 55) (size 0.8) (drill 0.4) (layers F.Cu B.Cu) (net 1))
 (via (at 79.9 54.8) (size 0.8) (drill 0.4) (layers F.Cu B.Cu) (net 1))
 (via (at 88.2 63.4) (size 0.8) (drill 0.4) (layers F.Cu B.Cu) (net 1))
 (via (at 87.5 70.4) (size 0.8) (drill 0.4) (layers F.Cu B.Cu) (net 1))
 (via (at 93.4 75.8) (size 0.8) (drill 0.4) (layers F.Cu B.Cu) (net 1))
 (via (at 84.4 73.9) (size 0.8) (drill 0.4) (layers F.Cu B.Cu) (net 1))
 (via (at 83.2 65.2) (size 0.8) (drill 0.4) (layers F.Cu B.Cu) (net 1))
 (via (at 93.1 81.7) (size 0.8) (drill 0.4) (layers F.Cu B.Cu) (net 1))
 (via (at 91.2 59.9) (size 0.8) (drill 0.4) (layers F.Cu B.Cu) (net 1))
 (via (at 82.6 50.4) (size 0.8) (drill 0.4) (layers F.Cu B.Cu) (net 1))
 (via (at 85 53.4) (size 0.8) (drill 0.4) (layers F.Cu B.Cu) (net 1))
 (via (at 91.4 54.1) (size 0.8) (drill 0.4) (layers F.Cu B.Cu) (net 1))
 (via (at 95.6 54.1) (size 0.8) (drill 0.4) (layers F.Cu B.Cu) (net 1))
 (via (at 96.3 59.1) (size 0.8) (drill 0.4) (layers F.Cu B.Cu) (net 1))
 (via (at 72 97.3) (size 0.8) (drill 0.4) (layers F.Cu B.Cu) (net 1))
 (via (at 75.1 92.2) (size 0.8) (drill 0.4) (layers F.Cu B.Cu) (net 1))
 (via (at 77.3 96.6) (size 0.8) (drill 0.4) (layers F.Cu B.Cu) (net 1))
 (via (at 77.4 103.5) (size 0.8) (drill 0.4) (layers F.Cu B.Cu) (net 1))
 (via (at 72.1 90.8) (size 0.8) (drill 0.4) (layers F.Cu B.Cu) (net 1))
 (via (at 100.3 53.3) (size 0.8) (drill 0.4) (layers F.Cu B.Cu) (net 1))
 (via (at 102.1 56.7) (size 0.8) (drill 0.4) (layers F.Cu B.Cu) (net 1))
 (segment (start 90 61.8) (end 90 65.1) (width 0.25) (layer B.Cu) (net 5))
 (segment (start 90 65.1) (end 90 65.1) (width 0.25) (layer B.Cu) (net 5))
 (via (at 90 65.1) (size 0.8) (drill 0.4) (layers F.Cu B.Cu) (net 5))
 (segment (start 94.36863 96.02) (end 94.34863 96) (width 0.25) (layer F.Cu) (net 5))
 (segment (start 95.5 96.02) (end 94.36863 96.02) (width 0.25) (layer F.Cu) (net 5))
 (segment (start 94.34863 96) (end 92.4 96) (width 0.25) (layer F.Cu) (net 5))
 (segment (start 90 93.6) (end 90 87) (width 0.25) (layer F.Cu) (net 5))
 (segment (start 92.4 96) (end 90 93.6) (width 0.25) (layer F.Cu) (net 5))
 (segment (start 90 65.1) (end 90 87) (width 0.25) (layer F.Cu) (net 5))
 (segment (start 90 87) (end 90 90.2) (width 0.25) (layer F.Cu) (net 5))
 (segment (start 53.57 59.89) (end 53.57 58.43) (width 0.25) (layer B.Cu) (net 5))
 (segment (start 53.57 58.43) (end 59 53) (width 0.25) (layer B.Cu) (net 5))
 (segment (start 81.2 53) (end 83.1 54.9) (width 0.25) (layer B.Cu) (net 5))
 (segment (start 59 53) (end 81.2 53) (width 0.25) (layer B.Cu) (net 5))
 (segment (start 82.4 54.2) (end 83.1 54.9) (width 0.25) (layer B.Cu) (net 5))
 (segment (start 83.1 54.9) (end 90 61.8) (width 0.25) (layer B.Cu) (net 5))
 (segment (start 73.2 56.6) (end 73.4 56.6) (width 0.25) (layer B.Cu) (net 19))
 (segment (start 78.8 56.6) (end 85.6 63.4) (width 0.25) (layer B.Cu) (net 19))
 (segment (start 85.6 63.4) (end 85.6 71.7) (width 0.25) (layer B.Cu) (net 19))
 (segment (start 92.14 78.24) (end 95.5 78.24) (width 0.25) (layer B.Cu) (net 19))
 (segment (start 85.6 71.7) (end 92.14 78.24) (width 0.25) (layer B.Cu) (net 19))
 (segment (start 61.4 56.6) (end 73.6 56.6) (width 0.25) (layer B.Cu) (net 19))
 (segment (start 55.57 62.43) (end 61.4 56.6) (width 0.25) (layer B.Cu) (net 19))
 (segment (start 53.57 62.43) (end 55.57 62.43) (width 0.25) (layer B.Cu) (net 19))
 (segment (start 73.2 56.6) (end 73.6 56.6) (width 0.25) (layer B.Cu) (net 19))
 (segment (start 73.6 56.6) (end 78.8 56.6) (width 0.25) (layer B.Cu) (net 19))
 (segment (start 71.41 92.91) (end 69.53 92.91) (width 1) (layer F.Cu) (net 26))
 (segment (start 74.6 96.1) (end 71.41 92.91) (width 1) (layer F.Cu) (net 26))
 (segment (start 74.6 98) (end 74.6 96.1) (width 1) (layer F.Cu) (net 26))
 (segment (start 80.26 101.1) (end 77.7 101.1) (width 1) (layer F.Cu) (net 26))
 (segment (start 77.7 101.1) (end 74.6 98) (width 1) (layer F.Cu) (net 26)))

